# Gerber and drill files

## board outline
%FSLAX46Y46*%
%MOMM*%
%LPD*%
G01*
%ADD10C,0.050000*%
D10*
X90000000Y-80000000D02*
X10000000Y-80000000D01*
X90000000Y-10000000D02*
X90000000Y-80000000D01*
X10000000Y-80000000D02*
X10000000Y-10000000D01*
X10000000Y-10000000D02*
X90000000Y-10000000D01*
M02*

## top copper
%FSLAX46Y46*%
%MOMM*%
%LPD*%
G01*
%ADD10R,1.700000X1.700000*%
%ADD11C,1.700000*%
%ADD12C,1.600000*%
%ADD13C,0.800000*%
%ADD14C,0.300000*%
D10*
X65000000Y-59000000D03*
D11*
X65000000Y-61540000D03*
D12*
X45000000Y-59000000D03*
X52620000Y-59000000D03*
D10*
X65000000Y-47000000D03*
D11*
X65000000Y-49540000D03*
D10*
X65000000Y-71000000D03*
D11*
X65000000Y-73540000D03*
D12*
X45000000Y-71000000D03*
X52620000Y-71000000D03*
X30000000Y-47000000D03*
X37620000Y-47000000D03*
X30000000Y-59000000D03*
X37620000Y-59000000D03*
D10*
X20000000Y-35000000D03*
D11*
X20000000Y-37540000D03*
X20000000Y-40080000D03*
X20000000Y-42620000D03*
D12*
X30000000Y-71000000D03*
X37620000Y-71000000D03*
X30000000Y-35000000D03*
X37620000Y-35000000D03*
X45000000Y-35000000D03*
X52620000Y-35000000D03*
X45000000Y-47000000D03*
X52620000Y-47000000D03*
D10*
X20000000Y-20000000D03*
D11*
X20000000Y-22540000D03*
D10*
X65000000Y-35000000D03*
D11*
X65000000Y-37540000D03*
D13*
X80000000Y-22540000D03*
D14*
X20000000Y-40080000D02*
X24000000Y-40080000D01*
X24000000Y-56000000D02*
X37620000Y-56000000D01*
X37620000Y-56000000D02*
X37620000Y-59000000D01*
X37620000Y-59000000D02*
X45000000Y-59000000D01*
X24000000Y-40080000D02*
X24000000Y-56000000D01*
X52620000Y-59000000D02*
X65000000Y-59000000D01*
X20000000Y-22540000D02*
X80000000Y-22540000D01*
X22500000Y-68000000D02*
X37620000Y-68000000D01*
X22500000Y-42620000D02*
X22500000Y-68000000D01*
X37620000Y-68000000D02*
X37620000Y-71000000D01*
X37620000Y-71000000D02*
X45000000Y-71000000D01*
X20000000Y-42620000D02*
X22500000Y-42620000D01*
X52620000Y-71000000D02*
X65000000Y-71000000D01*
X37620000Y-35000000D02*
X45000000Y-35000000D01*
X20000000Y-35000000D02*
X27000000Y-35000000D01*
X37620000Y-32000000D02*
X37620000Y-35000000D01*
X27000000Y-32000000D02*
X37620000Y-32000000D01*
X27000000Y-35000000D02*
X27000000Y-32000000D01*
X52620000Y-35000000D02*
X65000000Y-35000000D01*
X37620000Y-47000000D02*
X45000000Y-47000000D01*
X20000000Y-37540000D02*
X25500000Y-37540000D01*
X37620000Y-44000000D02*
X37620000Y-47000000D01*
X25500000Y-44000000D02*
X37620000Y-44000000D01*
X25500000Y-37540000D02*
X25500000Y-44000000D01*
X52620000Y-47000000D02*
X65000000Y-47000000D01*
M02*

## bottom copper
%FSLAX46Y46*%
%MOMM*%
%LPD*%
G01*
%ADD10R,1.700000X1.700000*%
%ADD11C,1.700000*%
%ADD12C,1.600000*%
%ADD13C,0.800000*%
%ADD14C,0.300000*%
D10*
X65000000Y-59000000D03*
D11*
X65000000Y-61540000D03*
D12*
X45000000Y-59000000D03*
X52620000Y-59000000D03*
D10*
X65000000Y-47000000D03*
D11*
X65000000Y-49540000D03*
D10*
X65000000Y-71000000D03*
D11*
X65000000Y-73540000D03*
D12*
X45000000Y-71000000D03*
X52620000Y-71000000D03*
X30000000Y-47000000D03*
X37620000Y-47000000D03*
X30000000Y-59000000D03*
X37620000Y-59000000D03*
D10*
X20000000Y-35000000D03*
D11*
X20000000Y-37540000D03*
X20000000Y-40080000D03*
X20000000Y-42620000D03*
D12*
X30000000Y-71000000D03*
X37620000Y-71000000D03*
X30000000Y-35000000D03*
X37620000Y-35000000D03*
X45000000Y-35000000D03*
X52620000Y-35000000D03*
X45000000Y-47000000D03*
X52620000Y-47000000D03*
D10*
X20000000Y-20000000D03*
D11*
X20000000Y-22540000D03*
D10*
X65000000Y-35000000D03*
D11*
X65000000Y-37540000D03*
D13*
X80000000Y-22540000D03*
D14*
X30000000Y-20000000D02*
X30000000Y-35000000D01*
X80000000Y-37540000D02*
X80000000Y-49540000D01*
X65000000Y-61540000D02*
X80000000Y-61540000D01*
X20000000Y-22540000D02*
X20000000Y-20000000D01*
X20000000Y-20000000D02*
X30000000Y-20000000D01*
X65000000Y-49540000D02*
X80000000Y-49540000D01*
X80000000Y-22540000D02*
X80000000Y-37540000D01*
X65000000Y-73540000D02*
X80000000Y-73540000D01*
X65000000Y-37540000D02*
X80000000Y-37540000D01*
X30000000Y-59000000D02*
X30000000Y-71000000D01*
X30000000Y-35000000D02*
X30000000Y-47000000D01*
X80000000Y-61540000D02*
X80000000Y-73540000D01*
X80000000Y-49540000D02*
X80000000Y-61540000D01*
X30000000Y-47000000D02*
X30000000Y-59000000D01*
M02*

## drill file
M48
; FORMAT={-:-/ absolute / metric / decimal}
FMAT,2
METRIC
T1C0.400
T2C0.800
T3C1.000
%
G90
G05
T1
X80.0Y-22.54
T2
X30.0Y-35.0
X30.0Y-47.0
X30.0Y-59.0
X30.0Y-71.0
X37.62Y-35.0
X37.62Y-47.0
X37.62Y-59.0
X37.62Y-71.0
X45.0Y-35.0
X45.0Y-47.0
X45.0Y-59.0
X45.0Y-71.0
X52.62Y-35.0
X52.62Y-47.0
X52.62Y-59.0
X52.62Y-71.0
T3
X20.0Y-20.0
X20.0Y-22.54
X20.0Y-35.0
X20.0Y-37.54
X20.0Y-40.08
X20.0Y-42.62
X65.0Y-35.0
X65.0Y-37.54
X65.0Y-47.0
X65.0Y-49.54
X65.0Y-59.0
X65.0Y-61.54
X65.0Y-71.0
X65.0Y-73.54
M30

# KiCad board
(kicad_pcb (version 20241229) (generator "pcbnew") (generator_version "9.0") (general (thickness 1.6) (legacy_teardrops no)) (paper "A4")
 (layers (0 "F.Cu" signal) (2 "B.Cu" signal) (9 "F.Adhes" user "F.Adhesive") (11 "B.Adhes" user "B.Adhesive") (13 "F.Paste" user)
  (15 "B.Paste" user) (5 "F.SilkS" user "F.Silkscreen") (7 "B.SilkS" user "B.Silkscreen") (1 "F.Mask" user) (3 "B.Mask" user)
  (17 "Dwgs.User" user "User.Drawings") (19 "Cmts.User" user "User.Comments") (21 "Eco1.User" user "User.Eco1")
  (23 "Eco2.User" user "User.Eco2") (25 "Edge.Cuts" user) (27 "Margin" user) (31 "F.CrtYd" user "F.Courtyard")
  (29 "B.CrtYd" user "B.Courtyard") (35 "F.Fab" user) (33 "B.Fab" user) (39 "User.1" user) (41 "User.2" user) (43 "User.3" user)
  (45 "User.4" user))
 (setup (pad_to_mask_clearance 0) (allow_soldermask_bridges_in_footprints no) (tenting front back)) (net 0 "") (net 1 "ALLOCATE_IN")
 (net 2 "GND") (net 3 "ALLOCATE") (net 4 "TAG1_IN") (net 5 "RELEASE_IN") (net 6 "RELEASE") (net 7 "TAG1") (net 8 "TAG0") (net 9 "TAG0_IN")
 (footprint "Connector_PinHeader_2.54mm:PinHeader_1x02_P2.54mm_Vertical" (layer "F.Cu") (at 65 59)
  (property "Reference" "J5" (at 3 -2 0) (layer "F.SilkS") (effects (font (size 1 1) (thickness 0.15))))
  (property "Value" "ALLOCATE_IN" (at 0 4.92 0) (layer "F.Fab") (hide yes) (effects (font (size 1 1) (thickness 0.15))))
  (pad "1" thru_hole rect (at 0 0) (size 1.7 1.7) (drill 1) (layers "*.Cu" "*.Mask") (remove_unused_layers no) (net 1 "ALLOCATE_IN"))
  (pad "2" thru_hole circle (at 0 2.54) (size 1.7 1.7) (drill 1) (layers "*.Cu" "*.Mask") (remove_unused_layers no) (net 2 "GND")))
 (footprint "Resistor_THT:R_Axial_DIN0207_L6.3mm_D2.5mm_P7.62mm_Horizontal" (layer "F.Cu") (at 45 59)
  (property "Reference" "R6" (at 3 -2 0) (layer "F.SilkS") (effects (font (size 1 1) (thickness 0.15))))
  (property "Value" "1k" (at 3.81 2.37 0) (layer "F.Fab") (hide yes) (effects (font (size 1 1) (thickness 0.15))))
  (pad "1" thru_hole circle (at 0 0) (size 1.6 1.6) (drill 0.8) (layers "*.Cu" "*.Mask") (remove_unused_layers no) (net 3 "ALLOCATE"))
  (pad "2" thru_hole circle (at 7.62 0) (size 1.6 1.6) (drill 0.8) (layers "*.Cu" "*.Mask") (remove_unused_layers no) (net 1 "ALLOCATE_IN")))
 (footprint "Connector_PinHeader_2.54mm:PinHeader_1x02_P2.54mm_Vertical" (layer "F.Cu") (at 65 47)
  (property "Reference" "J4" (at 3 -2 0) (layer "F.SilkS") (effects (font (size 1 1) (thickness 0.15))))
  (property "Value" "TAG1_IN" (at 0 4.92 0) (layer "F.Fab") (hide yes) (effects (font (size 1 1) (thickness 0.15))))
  (pad "1" thru_hole rect (at 0 0) (size 1.7 1.7) (drill 1) (layers "*.Cu" "*.Mask") (remove_unused_layers no) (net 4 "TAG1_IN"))
  (pad "2" thru_hole circle (at 0 2.54) (size 1.7 1.7) (drill 1) (layers "*.Cu" "*.Mask") (remove_unused_layers no) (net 2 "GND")))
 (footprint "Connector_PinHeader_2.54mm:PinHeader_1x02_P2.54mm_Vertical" (layer "F.Cu") (at 65 71)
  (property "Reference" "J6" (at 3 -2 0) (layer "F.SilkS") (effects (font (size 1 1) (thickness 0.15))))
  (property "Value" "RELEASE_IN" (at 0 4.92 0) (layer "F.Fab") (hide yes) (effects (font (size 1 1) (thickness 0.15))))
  (pad "1" thru_hole rect (at 0 0) (size 1.7 1.7) (drill 1) (layers "*.Cu" "*.Mask") (remove_unused_layers no) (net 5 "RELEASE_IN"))
  (pad "2" thru_hole circle (at 0 2.54) (size 1.7 1.7) (drill 1) (layers "*.Cu" "*.Mask") (remove_unused_layers no) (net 2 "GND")))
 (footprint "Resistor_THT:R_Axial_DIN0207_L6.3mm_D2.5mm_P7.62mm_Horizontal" (layer "F.Cu") (at 45 71)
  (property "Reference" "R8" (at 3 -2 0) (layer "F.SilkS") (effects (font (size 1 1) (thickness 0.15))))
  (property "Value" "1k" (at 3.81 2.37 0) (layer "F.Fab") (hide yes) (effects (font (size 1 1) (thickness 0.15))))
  (pad "1" thru_hole circle (at 0 0) (size 1.6 1.6) (drill 0.8) (layers "*.Cu" "*.Mask") (remove_unused_layers no) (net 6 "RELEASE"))
  (pad "2" thru_hole circle (at 7.62 0) (size 1.6 1.6) (drill 0.8) (layers "*.Cu" "*.Mask") (remove_unused_layers no) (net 5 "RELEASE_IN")))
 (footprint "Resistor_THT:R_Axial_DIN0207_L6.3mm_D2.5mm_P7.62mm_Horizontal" (layer "F.Cu") (at 30 47)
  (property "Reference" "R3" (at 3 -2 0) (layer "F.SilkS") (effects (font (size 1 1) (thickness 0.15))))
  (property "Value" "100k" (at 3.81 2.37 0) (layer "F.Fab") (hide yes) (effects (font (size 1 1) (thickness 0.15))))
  (pad "1" thru_hole circle (at 0 0) (size 1.6 1.6) (drill 0.8) (layers "*.Cu" "*.Mask") (remove_unused_layers no) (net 2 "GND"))
  (pad "2" thru_hole circle (at 7.62 0) (size 1.6 1.6) (drill 0.8) (layers "*.Cu" "*.Mask") (remove_unused_layers no) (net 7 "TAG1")))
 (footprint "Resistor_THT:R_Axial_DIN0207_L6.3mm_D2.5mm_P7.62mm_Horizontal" (layer "F.Cu") (at 30 59)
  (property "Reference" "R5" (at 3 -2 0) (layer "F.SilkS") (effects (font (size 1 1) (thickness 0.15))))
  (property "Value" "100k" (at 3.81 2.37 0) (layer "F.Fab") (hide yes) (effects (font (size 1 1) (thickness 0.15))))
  (pad "1" thru_hole circle (at 0 0) (size 1.6 1.6) (drill 0.8) (layers "*.Cu" "*.Mask") (remove_unused_layers no) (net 2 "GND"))
  (pad "2" thru_hole circle (at 7.62 0) (size 1.6 1.6) (drill 0.8) (layers "*.Cu" "*.Mask") (remove_unused_layers no) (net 3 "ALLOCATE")))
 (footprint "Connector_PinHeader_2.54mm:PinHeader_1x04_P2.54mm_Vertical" (layer "F.Cu") (at 20 35)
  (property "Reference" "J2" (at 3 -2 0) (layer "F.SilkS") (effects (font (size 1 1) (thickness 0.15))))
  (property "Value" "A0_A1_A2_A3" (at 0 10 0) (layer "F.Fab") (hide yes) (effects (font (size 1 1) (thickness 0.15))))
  (pad "1" thru_hole rect (at 0 0) (size 1.7 1.7) (drill 1) (layers "*.Cu" "*.Mask") (remove_unused_layers no) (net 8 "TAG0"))
  (pad "2" thru_hole circle (at 0 2.54) (size 1.7 1.7) (drill 1) (layers "*.Cu" "*.Mask") (remove_unused_layers no) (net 7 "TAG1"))
  (pad "3" thru_hole circle (at 0 5.08) (size 1.7 1.7) (drill 1) (layers "*.Cu" "*.Mask") (remove_unused_layers no) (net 3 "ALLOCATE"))
  (pad "4" thru_hole circle (at 0 7.62) (size 1.7 1.7) (drill 1) (layers "*.Cu" "*.Mask") (remove_unused_layers no) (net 6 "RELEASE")))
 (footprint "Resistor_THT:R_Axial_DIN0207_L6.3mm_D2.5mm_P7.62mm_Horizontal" (layer "F.Cu") (at 30 71)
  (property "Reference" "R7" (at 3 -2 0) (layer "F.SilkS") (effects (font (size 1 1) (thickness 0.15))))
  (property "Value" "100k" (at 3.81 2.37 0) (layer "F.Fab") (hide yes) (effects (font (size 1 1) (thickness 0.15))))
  (pad "1" thru_hole circle (at 0 0) (size 1.6 1.6) (drill 0.8) (layers "*.Cu" "*.Mask") (remove_unused_layers no) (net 2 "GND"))
  (pad "2" thru_hole circle (at 7.62 0) (size 1.6 1.6) (drill 0.8) (layers "*.Cu" "*.Mask") (remove_unused_layers no) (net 6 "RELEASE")))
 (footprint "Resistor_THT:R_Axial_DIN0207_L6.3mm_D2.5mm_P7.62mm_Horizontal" (layer "F.Cu") (at 30 35)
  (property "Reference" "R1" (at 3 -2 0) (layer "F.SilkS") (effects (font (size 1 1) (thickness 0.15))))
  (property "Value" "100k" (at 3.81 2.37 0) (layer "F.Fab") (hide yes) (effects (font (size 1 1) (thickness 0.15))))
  (pad "1" thru_hole circle (at 0 0) (size 1.6 1.6) (drill 0.8) (layers "*.Cu" "*.Mask") (remove_unused_layers no) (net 2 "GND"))
  (pad "2" thru_hole circle (at 7.62 0) (size 1.6 1.6) (drill 0.8) (layers "*.Cu" "*.Mask") (remove_unused_layers no) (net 8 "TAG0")))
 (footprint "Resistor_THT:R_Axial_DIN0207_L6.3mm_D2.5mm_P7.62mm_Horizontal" (layer "F.Cu") (at 45 35)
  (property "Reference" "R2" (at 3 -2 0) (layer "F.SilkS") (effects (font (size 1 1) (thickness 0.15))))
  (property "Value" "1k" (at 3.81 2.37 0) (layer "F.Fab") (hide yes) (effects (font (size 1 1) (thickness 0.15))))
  (pad "1" thru_hole circle (at 0 0) (size 1.6 1.6) (drill 0.8) (layers "*.Cu" "*.Mask") (remove_unused_layers no) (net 8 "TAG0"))
  (pad "2" thru_hole circle (at 7.62 0) (size 1.6 1.6) (drill 0.8) (layers "*.Cu" "*.Mask") (remove_unused_layers no) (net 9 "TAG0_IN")))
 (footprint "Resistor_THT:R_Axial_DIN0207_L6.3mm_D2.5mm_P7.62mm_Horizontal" (layer "F.Cu") (at 45 47)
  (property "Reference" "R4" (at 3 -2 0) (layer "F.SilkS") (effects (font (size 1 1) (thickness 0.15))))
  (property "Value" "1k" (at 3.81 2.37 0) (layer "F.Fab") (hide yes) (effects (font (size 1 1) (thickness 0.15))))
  (pad "1" thru_hole circle (at 0 0) (size 1.6 1.6) (drill 0.8) (layers "*.Cu" "*.Mask") (remove_unused_layers no) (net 7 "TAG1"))
  (pad "2" thru_hole circle (at 7.62 0) (size 1.6 1.6) (drill 0.8) (layers "*.Cu" "*.Mask") (remove_unused_layers no) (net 4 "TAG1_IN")))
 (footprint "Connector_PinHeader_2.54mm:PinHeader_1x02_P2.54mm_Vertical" (layer "F.Cu") (at 20 20)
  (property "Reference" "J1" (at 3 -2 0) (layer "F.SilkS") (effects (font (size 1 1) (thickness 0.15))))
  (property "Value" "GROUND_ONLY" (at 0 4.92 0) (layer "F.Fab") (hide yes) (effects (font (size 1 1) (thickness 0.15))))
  (pad "1" thru_hole rect (at 0 0) (size 1.7 1.7) (drill 1) (layers "*.Cu" "*.Mask") (remove_unused_layers no) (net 2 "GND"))
  (pad "2" thru_hole circle (at 0 2.54) (size 1.7 1.7) (drill 1) (layers "*.Cu" "*.Mask") (remove_unused_layers no) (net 2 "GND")))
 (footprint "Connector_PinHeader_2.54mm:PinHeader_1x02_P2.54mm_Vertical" (layer "F.Cu") (at 65 35)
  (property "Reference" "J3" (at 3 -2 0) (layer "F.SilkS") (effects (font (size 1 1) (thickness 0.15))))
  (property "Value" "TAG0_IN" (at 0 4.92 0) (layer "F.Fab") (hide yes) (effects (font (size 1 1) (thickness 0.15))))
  (pad "1" thru_hole rect (at 0 0) (size 1.7 1.7) (drill 1) (layers "*.Cu" "*.Mask") (remove_unused_layers no) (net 9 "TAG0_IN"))
  (pad "2" thru_hole circle (at 0 2.54) (size 1.7 1.7) (drill 1) (layers "*.Cu" "*.Mask") (remove_unused_layers no) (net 2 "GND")))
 (gr_line (start 90 80) (end 10 80) (stroke (width 0.05) (type default)) (layer "Edge.Cuts"))
 (gr_line (start 90 10) (end 90 80) (stroke (width 0.05) (type default)) (layer "Edge.Cuts"))
 (gr_line (start 10 80) (end 10 10) (stroke (width 0.05) (type default)) (layer "Edge.Cuts"))
 (gr_line (start 10 10) (end 90 10) (stroke (width 0.05) (type default)) (layer "Edge.Cuts"))
 (segment (start 20 40.08) (end 24 40.08) (width 0.3) (layer "F.Cu") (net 3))
 (segment (start 24 56) (end 37.62 56) (width 0.3) (layer "F.Cu") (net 3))
 (segment (start 37.62 56) (end 37.62 59) (width 0.3) (layer "F.Cu") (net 3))
 (segment (start 37.62 59) (end 45 59) (width 0.3) (layer "F.Cu") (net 3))
 (segment (start 24 40.08) (end 24 56) (width 0.3) (layer "F.Cu") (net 3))
 (segment (start 52.62 59) (end 65 59) (width 0.3) (layer "F.Cu") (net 1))
 (segment (start 20 22.54) (end 80 22.54) (width 0.3) (layer "F.Cu") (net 2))
 (via (at 80 22.54) (size 0.8) (drill 0.4) (layers "F.Cu" "B.Cu") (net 2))
 (segment (start 30 20) (end 30 35) (width 0.3) (layer "B.Cu") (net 2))
 (segment (start 80 37.54) (end 80 49.54) (width 0.3) (layer "B.Cu") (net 2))
 (segment (start 65 61.54) (end 80 61.54) (width 0.3) (layer "B.Cu") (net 2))
 (segment (start 20 22.54) (end 20 20) (width 0.3) (layer "B.Cu") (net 2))
 (segment (start 20 20) (end 30 20) (width 0.3) (layer "B.Cu") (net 2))
 (segment (start 65 49.54) (end 80 49.54) (width 0.3) (layer "B.Cu") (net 2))
 (segment (start 80 22.54) (end 80 37.54) (width 0.3) (layer "B.Cu") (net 2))
 (segment (start 65 73.54) (end 80 73.54) (width 0.3) (layer "B.Cu") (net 2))
 (segment (start 65 37.54) (end 80 37.54) (width 0.3) (layer "B.Cu") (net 2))
 (segment (start 30 59) (end 30 71) (width 0.3) (layer "B.Cu") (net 2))
 (segment (start 30 35) (end 30 47) (width 0.3) (layer "B.Cu") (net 2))
 (segment (start 80 61.54) (end 80 73.54) (width 0.3) (layer "B.Cu") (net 2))
 (segment (start 80 49.54) (end 80 61.54) (width 0.3) (layer "B.Cu") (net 2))
 (segment (start 30 47) (end 30 59) (width 0.3) (layer "B.Cu") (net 2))
 (segment (start 22.5 68) (end 37.62 68) (width 0.3) (layer "F.Cu") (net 6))
 (segment (start 22.5 42.62) (end 22.5 68) (width 0.3) (layer "F.Cu") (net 6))
 (segment (start 37.62 68) (end 37.62 71) (width 0.3) (layer "F.Cu") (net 6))
 (segment (start 37.62 71) (end 45 71) (width 0.3) (layer "F.Cu") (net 6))
 (segment (start 20 42.62) (end 22.5 42.62) (width 0.3) (layer "F.Cu") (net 6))
 (segment (start 52.62 71) (end 65 71) (width 0.3) (layer "F.Cu") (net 5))
 (segment (start 37.62 35) (end 45 35) (width 0.3) (layer "F.Cu") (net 8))
 (segment (start 20 35) (end 27 35) (width 0.3) (layer "F.Cu") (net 8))
 (segment (start 37.62 32) (end 37.62 35) (width 0.3) (layer "F.Cu") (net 8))
 (segment (start 27 32) (end 37.62 32) (width 0.3) (layer "F.Cu") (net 8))
 (segment (start 27 35) (end 27 32) (width 0.3) (layer "F.Cu") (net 8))
 (segment (start 52.62 35) (end 65 35) (width 0.3) (layer "F.Cu") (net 9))
 (segment (start 37.62 47) (end 45 47) (width 0.3) (layer "F.Cu") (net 7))
 (segment (start 20 37.54) (end 25.5 37.54) (width 0.3) (layer "F.Cu") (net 7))
 (segment (start 37.62 44) (end 37.62 47) (width 0.3) (layer "F.Cu") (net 7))
 (segment (start 25.5 44) (end 37.62 44) (width 0.3) (layer "F.Cu") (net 7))
 (segment (start 25.5 37.54) (end 25.5 44) (width 0.3) (layer "F.Cu") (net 7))
 (segment (start 52.62 47) (end 65 47) (width 0.3) (layer "F.Cu") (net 4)))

